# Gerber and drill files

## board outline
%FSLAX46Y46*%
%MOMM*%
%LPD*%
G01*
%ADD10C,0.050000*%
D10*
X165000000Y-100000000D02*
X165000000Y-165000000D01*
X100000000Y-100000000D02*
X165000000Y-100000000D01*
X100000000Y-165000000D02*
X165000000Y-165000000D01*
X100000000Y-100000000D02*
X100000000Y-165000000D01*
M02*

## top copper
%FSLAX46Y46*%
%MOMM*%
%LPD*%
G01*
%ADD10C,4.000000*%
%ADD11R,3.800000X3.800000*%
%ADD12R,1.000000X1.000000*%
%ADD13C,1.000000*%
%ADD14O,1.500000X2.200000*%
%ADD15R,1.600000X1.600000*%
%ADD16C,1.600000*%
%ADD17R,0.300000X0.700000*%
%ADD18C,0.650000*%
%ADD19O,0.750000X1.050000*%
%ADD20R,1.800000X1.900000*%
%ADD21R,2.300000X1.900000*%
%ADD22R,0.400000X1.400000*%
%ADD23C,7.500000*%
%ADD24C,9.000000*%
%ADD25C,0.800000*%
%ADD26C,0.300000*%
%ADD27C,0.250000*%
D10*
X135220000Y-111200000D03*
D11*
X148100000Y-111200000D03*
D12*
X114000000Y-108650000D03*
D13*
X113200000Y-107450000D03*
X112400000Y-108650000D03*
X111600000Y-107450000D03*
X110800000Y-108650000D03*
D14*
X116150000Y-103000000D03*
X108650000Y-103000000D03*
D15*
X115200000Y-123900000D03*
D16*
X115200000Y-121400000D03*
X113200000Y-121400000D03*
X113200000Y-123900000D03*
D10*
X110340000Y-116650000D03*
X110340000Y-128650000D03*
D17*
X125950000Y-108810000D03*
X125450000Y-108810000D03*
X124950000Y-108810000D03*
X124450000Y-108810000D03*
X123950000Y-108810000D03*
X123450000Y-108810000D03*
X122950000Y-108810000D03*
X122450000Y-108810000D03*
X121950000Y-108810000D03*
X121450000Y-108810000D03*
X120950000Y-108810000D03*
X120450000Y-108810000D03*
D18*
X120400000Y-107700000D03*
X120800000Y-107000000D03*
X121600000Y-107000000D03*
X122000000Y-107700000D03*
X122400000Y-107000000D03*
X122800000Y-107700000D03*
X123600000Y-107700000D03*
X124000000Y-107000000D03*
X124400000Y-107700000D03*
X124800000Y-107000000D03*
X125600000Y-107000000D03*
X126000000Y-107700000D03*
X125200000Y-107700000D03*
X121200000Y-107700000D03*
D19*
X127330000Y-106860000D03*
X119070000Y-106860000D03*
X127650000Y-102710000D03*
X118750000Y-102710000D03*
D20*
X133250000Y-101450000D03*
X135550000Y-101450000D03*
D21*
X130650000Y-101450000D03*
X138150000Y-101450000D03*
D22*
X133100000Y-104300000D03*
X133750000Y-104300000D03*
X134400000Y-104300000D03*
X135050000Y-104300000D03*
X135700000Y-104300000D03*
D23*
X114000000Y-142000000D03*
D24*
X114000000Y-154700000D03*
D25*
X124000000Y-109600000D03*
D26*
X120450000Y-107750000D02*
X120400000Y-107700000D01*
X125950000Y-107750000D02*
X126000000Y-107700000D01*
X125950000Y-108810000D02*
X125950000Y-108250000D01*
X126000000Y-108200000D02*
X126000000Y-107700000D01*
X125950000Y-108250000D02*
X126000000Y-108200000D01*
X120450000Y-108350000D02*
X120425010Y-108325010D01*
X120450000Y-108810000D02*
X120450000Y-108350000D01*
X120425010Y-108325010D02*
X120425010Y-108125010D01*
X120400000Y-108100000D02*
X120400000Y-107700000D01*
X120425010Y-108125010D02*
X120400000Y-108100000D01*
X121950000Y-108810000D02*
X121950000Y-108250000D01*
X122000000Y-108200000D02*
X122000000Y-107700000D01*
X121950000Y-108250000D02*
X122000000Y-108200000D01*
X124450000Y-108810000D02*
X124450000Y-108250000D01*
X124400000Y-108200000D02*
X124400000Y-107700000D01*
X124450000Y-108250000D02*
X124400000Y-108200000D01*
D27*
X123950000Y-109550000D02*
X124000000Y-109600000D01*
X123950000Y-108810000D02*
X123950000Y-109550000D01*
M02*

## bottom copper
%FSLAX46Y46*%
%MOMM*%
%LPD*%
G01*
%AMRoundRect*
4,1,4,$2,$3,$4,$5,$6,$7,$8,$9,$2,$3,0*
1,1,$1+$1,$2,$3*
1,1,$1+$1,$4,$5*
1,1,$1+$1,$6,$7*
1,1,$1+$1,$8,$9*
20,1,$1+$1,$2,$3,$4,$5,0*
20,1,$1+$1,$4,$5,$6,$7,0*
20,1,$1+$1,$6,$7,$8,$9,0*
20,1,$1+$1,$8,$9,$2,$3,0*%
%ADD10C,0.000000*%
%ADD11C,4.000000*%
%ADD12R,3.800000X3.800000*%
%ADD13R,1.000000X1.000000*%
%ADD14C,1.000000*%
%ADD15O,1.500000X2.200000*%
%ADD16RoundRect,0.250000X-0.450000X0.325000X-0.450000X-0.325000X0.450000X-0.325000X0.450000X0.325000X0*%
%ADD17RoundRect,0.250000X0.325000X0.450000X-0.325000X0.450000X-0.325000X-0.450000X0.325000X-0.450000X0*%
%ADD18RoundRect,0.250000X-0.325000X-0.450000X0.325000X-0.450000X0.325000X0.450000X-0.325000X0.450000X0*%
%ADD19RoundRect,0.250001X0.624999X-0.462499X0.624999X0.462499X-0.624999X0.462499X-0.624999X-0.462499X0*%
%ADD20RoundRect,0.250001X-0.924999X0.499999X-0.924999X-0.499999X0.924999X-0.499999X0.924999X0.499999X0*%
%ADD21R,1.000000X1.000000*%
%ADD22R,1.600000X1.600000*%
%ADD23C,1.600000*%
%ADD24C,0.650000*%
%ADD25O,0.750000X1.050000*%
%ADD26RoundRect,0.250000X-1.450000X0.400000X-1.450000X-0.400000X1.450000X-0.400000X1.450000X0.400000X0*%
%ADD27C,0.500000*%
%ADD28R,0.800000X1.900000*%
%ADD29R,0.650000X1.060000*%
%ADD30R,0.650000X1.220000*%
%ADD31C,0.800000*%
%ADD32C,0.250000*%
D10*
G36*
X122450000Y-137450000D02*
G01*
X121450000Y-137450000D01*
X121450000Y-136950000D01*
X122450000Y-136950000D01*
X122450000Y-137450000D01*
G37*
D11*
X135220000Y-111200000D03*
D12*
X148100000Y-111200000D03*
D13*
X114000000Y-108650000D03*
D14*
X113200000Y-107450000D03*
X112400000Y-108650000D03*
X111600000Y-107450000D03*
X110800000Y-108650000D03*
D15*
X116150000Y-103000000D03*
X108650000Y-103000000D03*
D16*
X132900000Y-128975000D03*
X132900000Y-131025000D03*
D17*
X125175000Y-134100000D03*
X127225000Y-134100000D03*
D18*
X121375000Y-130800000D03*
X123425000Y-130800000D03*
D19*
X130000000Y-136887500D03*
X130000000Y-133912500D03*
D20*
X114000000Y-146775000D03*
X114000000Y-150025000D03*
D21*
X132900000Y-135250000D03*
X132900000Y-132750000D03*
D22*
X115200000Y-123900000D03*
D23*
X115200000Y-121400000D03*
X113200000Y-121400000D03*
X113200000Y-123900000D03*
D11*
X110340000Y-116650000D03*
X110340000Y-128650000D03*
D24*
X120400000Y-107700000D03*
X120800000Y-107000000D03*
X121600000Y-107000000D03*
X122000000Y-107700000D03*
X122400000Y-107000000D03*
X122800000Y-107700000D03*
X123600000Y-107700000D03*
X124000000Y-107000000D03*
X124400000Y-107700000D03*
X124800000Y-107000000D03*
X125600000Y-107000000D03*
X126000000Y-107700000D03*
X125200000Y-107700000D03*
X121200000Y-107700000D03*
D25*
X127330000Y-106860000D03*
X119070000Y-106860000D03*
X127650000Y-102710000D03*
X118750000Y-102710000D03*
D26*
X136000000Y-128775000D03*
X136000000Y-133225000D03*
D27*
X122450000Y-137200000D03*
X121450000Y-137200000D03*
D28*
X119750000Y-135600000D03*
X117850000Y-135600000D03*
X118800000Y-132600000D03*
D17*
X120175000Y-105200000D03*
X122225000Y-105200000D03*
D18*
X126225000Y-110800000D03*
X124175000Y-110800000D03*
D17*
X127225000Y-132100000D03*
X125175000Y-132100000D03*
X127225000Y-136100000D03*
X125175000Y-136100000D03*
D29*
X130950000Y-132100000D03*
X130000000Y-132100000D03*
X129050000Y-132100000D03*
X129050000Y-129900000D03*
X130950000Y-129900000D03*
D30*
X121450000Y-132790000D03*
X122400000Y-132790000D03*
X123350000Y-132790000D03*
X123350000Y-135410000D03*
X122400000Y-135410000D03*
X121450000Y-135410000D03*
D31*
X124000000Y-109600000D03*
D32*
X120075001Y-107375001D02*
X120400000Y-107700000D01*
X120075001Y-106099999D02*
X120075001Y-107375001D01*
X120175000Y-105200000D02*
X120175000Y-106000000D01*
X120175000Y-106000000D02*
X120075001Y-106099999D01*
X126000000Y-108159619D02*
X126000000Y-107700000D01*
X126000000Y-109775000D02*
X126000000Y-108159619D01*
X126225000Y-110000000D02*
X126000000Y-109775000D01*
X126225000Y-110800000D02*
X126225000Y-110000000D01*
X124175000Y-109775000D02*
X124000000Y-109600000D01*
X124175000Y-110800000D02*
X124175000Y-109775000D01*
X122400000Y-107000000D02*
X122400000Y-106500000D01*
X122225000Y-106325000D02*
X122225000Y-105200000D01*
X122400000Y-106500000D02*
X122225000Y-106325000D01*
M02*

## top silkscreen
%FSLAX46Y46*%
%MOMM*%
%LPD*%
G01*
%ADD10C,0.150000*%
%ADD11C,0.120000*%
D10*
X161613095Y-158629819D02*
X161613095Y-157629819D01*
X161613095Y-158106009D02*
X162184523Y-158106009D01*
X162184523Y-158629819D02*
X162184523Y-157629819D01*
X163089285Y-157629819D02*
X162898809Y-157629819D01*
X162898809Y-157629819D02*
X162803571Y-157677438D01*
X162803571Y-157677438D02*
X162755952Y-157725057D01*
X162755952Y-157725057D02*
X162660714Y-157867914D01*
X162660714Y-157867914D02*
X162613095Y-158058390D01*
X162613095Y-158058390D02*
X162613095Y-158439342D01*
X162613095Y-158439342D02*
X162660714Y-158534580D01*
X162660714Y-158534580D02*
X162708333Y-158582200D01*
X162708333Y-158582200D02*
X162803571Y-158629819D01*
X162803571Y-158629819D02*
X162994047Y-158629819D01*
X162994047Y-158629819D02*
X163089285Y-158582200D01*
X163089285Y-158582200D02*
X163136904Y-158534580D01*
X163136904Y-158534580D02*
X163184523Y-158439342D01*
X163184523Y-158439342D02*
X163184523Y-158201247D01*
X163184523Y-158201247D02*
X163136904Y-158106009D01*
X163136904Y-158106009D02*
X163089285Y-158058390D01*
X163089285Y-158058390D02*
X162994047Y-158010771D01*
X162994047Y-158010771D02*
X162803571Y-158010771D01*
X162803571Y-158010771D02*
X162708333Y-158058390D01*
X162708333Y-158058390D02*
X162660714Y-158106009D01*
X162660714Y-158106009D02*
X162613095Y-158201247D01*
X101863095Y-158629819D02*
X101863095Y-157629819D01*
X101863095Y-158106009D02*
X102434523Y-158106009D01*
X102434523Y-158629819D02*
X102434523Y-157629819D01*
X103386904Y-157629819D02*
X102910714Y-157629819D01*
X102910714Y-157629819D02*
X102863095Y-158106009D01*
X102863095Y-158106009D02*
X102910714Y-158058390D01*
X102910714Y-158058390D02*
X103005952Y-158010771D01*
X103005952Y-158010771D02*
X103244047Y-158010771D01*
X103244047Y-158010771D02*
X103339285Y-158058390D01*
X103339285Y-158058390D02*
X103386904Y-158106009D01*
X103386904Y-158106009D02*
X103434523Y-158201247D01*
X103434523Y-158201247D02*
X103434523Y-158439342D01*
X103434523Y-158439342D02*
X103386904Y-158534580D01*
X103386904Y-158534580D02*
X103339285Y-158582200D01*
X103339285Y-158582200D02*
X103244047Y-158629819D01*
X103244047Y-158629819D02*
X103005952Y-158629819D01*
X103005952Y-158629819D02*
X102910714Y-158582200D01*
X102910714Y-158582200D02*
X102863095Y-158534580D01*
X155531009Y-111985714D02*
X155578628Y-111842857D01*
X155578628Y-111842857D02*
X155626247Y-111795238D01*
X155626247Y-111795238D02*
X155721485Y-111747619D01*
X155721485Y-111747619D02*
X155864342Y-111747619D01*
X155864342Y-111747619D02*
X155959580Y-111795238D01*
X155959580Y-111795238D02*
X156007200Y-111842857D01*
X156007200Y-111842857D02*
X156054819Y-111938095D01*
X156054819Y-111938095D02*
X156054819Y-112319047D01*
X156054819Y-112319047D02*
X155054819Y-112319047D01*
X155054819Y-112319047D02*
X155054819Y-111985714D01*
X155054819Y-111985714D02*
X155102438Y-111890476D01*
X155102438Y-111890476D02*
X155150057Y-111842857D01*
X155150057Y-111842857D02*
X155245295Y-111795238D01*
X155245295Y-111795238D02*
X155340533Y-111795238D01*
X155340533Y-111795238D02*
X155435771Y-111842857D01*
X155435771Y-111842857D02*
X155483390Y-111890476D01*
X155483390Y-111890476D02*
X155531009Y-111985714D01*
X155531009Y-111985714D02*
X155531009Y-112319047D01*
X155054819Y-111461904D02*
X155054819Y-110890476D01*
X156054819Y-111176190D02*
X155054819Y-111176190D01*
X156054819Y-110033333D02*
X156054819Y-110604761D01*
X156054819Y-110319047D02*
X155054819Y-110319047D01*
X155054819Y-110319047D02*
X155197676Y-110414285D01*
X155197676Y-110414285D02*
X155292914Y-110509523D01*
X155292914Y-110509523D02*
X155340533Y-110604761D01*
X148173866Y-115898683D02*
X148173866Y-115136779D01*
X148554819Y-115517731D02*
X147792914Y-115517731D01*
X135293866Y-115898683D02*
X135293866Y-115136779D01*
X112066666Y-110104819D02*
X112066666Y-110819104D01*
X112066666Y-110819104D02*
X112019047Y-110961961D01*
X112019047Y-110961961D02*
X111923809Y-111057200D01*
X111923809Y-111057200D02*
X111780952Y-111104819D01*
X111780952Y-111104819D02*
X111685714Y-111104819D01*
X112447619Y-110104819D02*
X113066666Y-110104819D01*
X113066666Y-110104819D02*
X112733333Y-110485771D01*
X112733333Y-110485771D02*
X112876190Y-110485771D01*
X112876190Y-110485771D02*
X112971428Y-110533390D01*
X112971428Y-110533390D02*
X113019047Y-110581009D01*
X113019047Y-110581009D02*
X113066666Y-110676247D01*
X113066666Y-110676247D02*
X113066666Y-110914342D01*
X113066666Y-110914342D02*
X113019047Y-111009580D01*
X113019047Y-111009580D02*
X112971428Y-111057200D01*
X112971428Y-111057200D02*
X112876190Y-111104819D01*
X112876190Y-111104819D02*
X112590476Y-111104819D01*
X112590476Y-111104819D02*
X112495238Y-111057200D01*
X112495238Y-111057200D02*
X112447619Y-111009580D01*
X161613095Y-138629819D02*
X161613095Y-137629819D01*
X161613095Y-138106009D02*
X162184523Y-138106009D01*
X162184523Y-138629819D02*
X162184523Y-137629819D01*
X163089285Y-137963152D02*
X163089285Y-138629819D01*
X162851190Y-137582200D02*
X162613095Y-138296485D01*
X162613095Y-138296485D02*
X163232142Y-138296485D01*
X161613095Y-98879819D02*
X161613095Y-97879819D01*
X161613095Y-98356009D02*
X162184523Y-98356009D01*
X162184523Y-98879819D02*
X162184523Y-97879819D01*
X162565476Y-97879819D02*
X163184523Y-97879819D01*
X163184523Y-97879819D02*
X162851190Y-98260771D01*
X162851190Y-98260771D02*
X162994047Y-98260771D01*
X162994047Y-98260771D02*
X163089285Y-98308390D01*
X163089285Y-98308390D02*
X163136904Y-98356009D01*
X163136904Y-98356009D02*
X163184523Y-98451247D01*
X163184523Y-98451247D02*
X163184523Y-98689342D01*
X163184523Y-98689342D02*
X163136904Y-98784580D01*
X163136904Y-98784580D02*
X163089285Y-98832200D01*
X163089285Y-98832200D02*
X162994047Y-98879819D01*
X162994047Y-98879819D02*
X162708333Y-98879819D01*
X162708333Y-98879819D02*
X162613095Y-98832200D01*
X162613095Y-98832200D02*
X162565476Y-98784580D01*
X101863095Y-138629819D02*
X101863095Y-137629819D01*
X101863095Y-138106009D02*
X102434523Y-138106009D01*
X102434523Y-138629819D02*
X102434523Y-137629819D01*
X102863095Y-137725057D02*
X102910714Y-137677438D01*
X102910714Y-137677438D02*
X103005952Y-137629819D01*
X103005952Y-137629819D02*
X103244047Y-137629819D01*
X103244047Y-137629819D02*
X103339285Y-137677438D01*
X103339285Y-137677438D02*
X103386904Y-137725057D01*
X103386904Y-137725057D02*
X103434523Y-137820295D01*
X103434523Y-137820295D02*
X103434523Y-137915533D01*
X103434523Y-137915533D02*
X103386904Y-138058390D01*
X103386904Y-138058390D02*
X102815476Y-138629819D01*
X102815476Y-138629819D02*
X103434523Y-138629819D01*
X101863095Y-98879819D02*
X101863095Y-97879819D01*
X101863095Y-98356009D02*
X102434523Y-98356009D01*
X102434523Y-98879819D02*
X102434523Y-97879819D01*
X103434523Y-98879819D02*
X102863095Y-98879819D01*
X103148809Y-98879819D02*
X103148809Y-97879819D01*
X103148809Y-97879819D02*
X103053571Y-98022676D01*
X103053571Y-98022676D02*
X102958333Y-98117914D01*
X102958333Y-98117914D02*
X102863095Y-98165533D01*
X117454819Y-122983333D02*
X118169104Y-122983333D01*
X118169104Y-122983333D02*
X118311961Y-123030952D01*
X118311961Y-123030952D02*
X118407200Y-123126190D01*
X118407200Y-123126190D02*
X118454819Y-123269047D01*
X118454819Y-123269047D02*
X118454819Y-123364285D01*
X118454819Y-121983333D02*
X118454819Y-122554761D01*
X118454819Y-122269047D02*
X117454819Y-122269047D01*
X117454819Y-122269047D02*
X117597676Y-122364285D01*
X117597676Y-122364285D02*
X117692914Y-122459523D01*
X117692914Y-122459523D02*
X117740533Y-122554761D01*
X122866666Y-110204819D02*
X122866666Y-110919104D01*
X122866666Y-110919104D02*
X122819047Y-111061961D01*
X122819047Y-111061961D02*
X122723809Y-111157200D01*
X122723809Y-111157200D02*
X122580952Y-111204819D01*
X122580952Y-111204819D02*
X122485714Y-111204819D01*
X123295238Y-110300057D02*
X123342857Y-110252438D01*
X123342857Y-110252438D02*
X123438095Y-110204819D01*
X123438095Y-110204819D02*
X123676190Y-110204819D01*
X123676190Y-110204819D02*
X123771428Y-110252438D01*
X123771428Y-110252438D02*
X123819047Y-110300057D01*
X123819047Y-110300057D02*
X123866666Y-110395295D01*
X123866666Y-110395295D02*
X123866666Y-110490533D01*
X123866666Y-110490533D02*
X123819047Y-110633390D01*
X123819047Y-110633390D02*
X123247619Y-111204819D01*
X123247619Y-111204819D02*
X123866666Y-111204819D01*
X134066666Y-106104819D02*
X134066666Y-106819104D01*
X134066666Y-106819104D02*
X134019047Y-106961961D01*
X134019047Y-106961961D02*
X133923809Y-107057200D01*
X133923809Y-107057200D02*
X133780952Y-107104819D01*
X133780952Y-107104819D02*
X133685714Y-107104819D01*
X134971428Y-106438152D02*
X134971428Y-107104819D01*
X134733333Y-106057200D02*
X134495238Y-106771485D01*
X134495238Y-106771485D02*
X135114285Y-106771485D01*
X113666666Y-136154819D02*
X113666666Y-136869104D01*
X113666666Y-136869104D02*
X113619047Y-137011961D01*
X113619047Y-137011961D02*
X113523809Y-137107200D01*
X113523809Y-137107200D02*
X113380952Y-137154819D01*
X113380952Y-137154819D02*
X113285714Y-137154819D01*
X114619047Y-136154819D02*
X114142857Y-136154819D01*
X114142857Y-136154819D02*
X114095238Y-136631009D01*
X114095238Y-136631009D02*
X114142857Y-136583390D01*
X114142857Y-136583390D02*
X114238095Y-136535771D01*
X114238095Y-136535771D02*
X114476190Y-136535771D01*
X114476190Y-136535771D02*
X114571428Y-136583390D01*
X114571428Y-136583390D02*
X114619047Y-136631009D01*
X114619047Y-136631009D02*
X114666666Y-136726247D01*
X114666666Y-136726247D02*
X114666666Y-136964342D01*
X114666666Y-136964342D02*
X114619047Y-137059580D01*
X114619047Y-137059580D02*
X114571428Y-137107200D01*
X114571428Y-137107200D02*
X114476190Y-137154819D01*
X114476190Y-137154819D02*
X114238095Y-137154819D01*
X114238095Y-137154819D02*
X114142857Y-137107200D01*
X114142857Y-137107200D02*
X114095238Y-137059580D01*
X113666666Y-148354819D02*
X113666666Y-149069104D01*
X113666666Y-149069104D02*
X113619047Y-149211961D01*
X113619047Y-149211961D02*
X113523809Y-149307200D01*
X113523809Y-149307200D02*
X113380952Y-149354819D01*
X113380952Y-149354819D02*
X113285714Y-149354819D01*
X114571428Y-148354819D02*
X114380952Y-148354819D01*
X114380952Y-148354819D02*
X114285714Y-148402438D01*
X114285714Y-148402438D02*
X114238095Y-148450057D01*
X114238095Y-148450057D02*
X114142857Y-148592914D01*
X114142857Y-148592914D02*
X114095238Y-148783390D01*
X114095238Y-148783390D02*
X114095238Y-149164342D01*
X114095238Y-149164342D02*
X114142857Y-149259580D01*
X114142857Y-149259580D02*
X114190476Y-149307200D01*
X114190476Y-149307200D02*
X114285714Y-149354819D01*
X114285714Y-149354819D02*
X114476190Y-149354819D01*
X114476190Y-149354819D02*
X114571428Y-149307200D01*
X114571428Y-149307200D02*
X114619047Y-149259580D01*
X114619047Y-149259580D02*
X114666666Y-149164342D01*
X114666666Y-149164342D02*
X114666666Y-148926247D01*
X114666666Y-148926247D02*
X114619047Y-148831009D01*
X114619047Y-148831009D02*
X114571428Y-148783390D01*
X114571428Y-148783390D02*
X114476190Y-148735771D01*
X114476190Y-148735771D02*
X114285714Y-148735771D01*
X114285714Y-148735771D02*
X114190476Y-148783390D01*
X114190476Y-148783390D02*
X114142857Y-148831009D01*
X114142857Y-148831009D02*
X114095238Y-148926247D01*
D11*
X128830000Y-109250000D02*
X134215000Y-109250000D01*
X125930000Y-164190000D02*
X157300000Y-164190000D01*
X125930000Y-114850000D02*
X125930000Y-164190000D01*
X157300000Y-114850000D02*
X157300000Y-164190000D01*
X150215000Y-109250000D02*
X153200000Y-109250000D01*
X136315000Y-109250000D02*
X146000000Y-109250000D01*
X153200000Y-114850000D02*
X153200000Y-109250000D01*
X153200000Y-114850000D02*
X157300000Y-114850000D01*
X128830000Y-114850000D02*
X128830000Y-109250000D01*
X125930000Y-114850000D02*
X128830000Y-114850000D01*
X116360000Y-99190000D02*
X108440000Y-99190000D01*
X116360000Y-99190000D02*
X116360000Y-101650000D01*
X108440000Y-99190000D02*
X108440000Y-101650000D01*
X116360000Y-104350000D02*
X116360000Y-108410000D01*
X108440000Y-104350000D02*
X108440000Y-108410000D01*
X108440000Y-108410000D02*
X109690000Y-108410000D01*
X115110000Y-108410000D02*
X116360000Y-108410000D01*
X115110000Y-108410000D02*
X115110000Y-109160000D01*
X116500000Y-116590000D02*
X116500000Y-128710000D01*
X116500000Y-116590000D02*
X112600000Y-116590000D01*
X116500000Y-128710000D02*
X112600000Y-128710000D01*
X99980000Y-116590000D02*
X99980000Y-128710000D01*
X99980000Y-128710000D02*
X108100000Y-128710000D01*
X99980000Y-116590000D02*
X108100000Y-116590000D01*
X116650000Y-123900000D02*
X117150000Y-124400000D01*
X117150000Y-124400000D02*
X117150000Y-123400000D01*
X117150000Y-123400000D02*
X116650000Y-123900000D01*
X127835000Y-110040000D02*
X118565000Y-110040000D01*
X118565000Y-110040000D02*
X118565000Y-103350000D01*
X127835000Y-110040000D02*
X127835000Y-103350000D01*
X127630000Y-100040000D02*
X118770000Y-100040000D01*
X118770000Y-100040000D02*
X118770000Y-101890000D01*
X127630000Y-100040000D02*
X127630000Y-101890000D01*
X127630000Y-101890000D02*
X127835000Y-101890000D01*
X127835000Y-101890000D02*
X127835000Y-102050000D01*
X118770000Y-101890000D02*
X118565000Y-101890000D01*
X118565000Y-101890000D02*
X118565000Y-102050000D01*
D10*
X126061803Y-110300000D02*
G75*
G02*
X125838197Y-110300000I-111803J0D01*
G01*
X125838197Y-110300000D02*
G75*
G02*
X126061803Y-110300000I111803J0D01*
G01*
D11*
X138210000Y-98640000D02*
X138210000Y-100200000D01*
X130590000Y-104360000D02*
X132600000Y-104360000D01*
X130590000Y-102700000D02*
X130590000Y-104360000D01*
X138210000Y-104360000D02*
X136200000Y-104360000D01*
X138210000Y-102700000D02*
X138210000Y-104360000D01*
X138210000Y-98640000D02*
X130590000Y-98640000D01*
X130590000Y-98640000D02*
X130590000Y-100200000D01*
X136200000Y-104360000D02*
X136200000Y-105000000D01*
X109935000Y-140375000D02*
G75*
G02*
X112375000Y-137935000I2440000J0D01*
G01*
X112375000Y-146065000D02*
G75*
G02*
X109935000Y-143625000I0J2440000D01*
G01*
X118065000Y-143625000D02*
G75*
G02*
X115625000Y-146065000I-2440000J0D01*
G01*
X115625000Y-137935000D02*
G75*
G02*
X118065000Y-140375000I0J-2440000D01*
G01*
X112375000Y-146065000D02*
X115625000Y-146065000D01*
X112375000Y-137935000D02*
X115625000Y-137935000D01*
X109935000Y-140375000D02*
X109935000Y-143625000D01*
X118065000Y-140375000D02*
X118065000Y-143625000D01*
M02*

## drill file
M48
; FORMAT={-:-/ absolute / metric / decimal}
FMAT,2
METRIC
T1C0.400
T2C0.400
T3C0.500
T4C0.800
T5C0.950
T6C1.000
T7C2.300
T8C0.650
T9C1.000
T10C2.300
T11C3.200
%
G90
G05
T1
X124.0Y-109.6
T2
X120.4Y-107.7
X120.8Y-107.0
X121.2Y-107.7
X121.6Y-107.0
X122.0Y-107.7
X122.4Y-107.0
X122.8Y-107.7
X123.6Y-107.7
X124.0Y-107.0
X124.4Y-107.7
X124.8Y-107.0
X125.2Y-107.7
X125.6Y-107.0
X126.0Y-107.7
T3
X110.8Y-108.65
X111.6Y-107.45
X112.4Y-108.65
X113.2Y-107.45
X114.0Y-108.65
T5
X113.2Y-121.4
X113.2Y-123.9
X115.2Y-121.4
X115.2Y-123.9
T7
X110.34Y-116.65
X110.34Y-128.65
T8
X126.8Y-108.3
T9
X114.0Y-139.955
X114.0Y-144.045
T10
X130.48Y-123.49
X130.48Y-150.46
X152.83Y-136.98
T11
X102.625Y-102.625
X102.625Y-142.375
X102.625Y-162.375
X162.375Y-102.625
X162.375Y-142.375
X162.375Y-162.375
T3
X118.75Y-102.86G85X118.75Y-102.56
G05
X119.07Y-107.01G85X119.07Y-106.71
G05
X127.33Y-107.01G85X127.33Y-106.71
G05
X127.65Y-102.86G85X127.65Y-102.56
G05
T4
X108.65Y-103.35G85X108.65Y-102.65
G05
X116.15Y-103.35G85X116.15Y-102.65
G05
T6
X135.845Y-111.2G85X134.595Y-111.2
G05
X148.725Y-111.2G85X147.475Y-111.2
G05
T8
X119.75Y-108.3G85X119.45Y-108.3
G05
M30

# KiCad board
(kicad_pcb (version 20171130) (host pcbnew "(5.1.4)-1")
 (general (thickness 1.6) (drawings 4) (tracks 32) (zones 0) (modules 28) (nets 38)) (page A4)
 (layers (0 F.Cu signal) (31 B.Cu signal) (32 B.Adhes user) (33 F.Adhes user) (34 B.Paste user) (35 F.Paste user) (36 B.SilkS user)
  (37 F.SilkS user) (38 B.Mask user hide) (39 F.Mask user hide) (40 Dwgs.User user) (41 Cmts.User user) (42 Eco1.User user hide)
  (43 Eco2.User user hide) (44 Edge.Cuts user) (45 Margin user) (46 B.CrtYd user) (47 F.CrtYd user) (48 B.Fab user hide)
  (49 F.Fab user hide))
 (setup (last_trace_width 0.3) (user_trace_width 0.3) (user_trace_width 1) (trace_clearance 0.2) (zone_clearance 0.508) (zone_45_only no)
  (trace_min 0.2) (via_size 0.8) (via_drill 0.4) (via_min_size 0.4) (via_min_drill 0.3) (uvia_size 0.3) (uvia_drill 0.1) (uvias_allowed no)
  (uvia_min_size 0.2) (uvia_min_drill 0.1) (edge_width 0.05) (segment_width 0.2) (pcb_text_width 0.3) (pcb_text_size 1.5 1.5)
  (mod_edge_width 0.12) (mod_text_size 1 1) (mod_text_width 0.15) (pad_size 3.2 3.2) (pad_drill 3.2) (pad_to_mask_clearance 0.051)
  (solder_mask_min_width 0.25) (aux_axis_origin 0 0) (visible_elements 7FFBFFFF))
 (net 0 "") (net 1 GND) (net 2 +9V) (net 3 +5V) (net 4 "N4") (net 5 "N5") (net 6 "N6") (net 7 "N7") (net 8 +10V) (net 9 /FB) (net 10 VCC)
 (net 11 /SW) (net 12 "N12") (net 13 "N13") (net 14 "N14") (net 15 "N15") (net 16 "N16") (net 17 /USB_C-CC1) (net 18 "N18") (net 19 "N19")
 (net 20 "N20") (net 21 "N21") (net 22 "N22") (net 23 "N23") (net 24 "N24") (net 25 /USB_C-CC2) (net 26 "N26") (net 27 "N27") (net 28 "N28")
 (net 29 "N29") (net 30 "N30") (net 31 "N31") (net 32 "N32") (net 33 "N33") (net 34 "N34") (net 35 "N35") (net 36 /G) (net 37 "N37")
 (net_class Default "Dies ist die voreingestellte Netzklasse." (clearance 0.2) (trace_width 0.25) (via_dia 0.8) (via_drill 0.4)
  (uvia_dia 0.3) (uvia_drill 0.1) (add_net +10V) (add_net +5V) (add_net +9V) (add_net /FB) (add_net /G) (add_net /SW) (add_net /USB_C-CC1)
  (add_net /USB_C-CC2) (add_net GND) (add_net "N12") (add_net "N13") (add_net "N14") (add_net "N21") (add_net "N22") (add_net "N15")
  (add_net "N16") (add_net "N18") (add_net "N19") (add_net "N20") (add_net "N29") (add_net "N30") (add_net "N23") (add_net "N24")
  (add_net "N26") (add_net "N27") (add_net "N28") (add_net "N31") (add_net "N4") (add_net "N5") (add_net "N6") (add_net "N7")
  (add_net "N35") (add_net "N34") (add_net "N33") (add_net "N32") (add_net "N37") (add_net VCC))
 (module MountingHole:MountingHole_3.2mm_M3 (layer F.Cu) (at 162.375 162.375)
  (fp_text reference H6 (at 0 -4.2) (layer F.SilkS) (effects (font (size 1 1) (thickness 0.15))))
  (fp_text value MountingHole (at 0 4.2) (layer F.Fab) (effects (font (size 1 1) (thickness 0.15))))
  (pad 1 np_thru_hole circle (at 0 0) (size 3.2 3.2) (drill 3.2) (layers *.Cu *.Mask)))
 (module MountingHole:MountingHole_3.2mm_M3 (layer F.Cu) (at 102.625 162.375)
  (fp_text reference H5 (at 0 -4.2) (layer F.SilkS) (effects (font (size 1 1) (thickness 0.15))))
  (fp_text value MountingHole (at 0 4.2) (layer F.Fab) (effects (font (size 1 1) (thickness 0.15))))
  (pad 1 np_thru_hole circle (at 0 0) (size 3.2 3.2) (drill 3.2) (layers *.Cu *.Mask)))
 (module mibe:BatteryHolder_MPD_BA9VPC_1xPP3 (layer F.Cu) (at 148.1 111.2 270)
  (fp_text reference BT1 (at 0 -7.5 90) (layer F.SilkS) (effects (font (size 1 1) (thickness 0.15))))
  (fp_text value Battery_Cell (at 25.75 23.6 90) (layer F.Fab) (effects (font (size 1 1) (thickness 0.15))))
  (fp_line (start -1.95 19.27) (end -1.95 13.885) (layer F.SilkS) (width 0.12))
  (fp_line (start 52.99 22.17) (end 52.99 -9.2) (layer F.SilkS) (width 0.12))
  (fp_line (start 3.65 22.17) (end 52.99 22.17) (layer F.SilkS) (width 0.12))
  (fp_line (start 3.65 -9.2) (end 52.99 -9.2) (layer F.SilkS) (width 0.12))
  (fp_line (start -1.95 -2.115) (end -1.95 -5.1) (layer F.SilkS) (width 0.12))
  (fp_line (start -1.95 11.785) (end -1.95 2.1) (layer F.SilkS) (width 0.12))
  (fp_line (start 3.65 -5.1) (end -1.95 -5.1) (layer F.SilkS) (width 0.12))
  (fp_line (start 3.65 -5.1) (end 3.65 -9.2) (layer F.SilkS) (width 0.12))
  (fp_line (start 3.65 19.27) (end -1.95 19.27) (layer F.SilkS) (width 0.12))
  (fp_line (start 3.65 22.17) (end 3.65 19.27) (layer F.SilkS) (width 0.12))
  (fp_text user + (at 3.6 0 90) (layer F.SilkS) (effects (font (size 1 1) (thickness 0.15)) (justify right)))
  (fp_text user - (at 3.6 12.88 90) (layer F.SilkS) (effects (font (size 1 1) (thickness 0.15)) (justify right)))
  (pad "" np_thru_hole circle (at 39.26 17.62 270) (size 2.3 2.3) (drill 2.3) (layers *.Cu *.Mask))
  (pad "" np_thru_hole circle (at 12.29 17.62 270) (size 2.3 2.3) (drill 2.3) (layers *.Cu *.Mask))
  (pad "" np_thru_hole circle (at 25.78 -4.73 270) (size 2.3 2.3) (drill 2.3) (layers *.Cu *.Mask))
  (pad 2 thru_hole circle (at 0 12.88 270) (size 4 4) (drill oval 1 2.25) (layers *.Cu *.Mask) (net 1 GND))
  (pad 1 thru_hole rect (at 0 0 270) (size 3.8 3.8) (drill oval 1 2.25) (layers *.Cu *.Mask) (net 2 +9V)))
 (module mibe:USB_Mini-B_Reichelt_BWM (layer F.Cu) (at 114 108.65 180)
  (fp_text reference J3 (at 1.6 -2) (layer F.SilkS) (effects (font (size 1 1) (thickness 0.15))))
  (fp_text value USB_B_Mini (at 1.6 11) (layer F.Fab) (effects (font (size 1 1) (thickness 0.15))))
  (fp_line (start -2.36 9.46) (end 5.56 9.46) (layer F.SilkS) (width 0.12))
  (fp_line (start -2.36 9.46) (end -2.36 7) (layer F.SilkS) (width 0.12))
  (fp_line (start 5.56 9.46) (end 5.56 7) (layer F.SilkS) (width 0.12))
  (fp_line (start -2.36 4.3) (end -2.36 0.24) (layer F.SilkS) (width 0.12))
  (fp_line (start 5.56 4.3) (end 5.56 0.24) (layer F.SilkS) (width 0.12))
  (fp_line (start 5.56 0.24) (end 4.31 0.24) (layer F.SilkS) (width 0.12))
  (fp_line (start -1.11 0.24) (end -2.36 0.24) (layer F.SilkS) (width 0.12))
  (fp_line (start -1.11 0.24) (end -1.11 -0.51) (layer F.SilkS) (width 0.12))
  (pad 1 thru_hole rect (at 0 0 180) (size 1 1) (drill 0.5) (layers *.Cu *.Mask) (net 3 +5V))
  (pad 2 thru_hole circle (at 0.8 1.2 180) (size 1 1) (drill 0.5) (layers *.Cu *.Mask) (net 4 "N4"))
  (pad 3 thru_hole circle (at 1.6 0 180) (size 1 1) (drill 0.5) (layers *.Cu *.Mask) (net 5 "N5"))
  (pad 4 thru_hole circle (at 2.4 1.2 180) (size 1 1) (drill 0.5) (layers *.Cu *.Mask) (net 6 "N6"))
  (pad 5 thru_hole circle (at 3.2 0 180) (size 1 1) (drill 0.5) (layers *.Cu *.Mask) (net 1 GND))
  (pad 6 thru_hole oval (at -2.15 5.65 180) (size 1.5 2.2) (drill oval 0.8 1.5) (layers *.Cu *.Mask) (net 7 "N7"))
  (pad 6 thru_hole oval (at 5.35 5.65 180) (size 1.5 2.2) (drill oval 0.8 1.5) (layers *.Cu *.Mask) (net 7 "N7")))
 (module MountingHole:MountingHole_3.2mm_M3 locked (layer F.Cu) (at 162.375 142.375)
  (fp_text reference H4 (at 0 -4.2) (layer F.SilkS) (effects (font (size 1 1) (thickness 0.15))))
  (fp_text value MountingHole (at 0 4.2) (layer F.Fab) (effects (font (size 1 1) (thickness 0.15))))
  (pad 1 np_thru_hole circle (at 0 0) (size 3.2 3.2) (drill 3.2) (layers *.Cu *.Mask)))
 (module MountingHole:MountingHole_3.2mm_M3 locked (layer F.Cu) (at 162.375 102.625)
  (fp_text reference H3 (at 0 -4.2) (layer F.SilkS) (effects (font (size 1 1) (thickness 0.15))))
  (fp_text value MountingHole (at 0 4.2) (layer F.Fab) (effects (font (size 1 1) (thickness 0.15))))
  (pad 1 np_thru_hole circle (at 0 0) (size 3.2 3.2) (drill 3.2) (layers *.Cu *.Mask)))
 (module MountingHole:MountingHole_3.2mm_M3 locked (layer F.Cu) (at 102.625 142.375)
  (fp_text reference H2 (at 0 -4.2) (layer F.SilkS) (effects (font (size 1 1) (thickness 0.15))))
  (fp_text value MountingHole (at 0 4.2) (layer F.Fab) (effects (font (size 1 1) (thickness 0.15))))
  (pad 1 np_thru_hole circle (at 0 0) (size 3.2 3.2) (drill 3.2) (layers *.Cu *.Mask)))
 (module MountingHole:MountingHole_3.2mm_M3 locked (layer F.Cu) (at 102.625 102.625)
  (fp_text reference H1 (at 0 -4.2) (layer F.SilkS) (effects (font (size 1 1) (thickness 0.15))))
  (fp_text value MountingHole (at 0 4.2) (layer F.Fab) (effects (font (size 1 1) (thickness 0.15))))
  (pad 1 np_thru_hole circle (at 0 0) (size 3.2 3.2) (drill 3.2) (layers *.Cu *.Mask)))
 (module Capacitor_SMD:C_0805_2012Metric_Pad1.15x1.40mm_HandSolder (layer B.Cu) (at 132.9 130 270)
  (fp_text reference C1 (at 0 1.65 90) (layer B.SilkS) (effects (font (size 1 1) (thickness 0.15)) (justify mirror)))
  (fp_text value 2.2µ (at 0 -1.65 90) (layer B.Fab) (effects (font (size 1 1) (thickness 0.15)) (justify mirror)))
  (pad 1 smd roundrect (at -1.025 0 270) (size 1.15 1.4) (layers B.Cu B.Paste B.Mask) (roundrect_rratio 0.217391) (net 3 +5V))
  (pad 2 smd roundrect (at 1.025 0 270) (size 1.15 1.4) (layers B.Cu B.Paste B.Mask) (roundrect_rratio 0.217391) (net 1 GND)))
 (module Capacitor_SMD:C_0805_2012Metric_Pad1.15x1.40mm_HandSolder (layer B.Cu) (at 126.2 134.1 180)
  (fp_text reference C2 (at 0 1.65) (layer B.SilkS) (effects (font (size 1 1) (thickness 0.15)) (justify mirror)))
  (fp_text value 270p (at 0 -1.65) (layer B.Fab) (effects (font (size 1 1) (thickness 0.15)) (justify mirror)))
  (pad 2 smd roundrect (at 1.025 0 180) (size 1.15 1.4) (layers B.Cu B.Paste B.Mask) (roundrect_rratio 0.217391) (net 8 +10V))
  (pad 1 smd roundrect (at -1.025 0 180) (size 1.15 1.4) (layers B.Cu B.Paste B.Mask) (roundrect_rratio 0.217391) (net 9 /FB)))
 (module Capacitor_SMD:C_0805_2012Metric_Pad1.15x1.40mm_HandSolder (layer B.Cu) (at 122.4 130.8)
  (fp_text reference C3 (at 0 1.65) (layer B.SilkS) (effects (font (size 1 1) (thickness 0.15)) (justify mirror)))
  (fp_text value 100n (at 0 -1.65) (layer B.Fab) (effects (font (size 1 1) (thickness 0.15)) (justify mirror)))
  (pad 1 smd roundrect (at -1.025 0) (size 1.15 1.4) (layers B.Cu B.Paste B.Mask) (roundrect_rratio 0.217391) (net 2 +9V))
  (pad 2 smd roundrect (at 1.025 0) (size 1.15 1.4) (layers B.Cu B.Paste B.Mask) (roundrect_rratio 0.217391) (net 1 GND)))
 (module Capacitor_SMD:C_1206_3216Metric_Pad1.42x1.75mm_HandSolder (layer B.Cu) (at 130 135.4 90)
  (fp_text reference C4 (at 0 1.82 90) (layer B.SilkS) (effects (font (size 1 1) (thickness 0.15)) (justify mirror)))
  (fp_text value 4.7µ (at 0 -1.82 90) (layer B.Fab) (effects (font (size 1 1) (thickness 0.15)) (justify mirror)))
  (pad 1 smd roundrect (at -1.4875 0 90) (size 1.425 1.75) (layers B.Cu B.Paste B.Mask) (roundrect_rratio 0.175439) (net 8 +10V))
  (pad 2 smd roundrect (at 1.4875 0 90) (size 1.425 1.75) (layers B.Cu B.Paste B.Mask) (roundrect_rratio 0.175439) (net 1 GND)))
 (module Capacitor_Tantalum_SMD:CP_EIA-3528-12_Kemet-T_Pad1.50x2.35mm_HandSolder (layer B.Cu) (at 114 148.4 270)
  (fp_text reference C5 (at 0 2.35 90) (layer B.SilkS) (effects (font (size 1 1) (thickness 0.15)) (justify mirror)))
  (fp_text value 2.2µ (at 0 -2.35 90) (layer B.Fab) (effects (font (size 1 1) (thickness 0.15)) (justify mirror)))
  (pad 1 smd roundrect (at -1.625 0 270) (size 1.5 2.35) (layers B.Cu B.Paste B.Mask) (roundrect_rratio 0.166667) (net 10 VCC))
  (pad 2 smd roundrect (at 1.625 0 270) (size 1.5 2.35) (layers B.Cu B.Paste B.Mask) (roundrect_rratio 0.166667) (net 1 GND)))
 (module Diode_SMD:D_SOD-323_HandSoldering (layer B.Cu) (at 132.9 134 90)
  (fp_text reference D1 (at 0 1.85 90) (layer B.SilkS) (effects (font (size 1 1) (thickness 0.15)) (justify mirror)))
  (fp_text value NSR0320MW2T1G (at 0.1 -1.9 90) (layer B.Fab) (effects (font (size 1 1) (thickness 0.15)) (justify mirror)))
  (pad 1 smd rect (at -1.25 0 90) (size 1 1) (layers B.Cu B.Paste B.Mask) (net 8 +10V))
  (pad 2 smd rect (at 1.25 0 90) (size 1 1) (layers B.Cu B.Paste B.Mask) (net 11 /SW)))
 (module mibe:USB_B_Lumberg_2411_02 (layer F.Cu) (at 115.2 123.9 270)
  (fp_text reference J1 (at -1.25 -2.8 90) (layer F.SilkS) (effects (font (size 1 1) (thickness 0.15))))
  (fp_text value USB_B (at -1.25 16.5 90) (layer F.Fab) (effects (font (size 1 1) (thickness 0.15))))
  (fp_line (start -7.31 -1.3) (end 4.81 -1.3) (layer F.SilkS) (width 0.12))
  (fp_line (start -7.31 -1.3) (end -7.31 2.6) (layer F.SilkS) (width 0.12))
  (fp_line (start 4.81 -1.3) (end 4.81 2.6) (layer F.SilkS) (width 0.12))
  (fp_line (start -7.31 15.22) (end 4.81 15.22) (layer F.SilkS) (width 0.12))
  (fp_line (start 4.81 15.22) (end 4.81 7.1) (layer F.SilkS) (width 0.12))
  (fp_line (start -7.31 15.22) (end -7.31 7.1) (layer F.SilkS) (width 0.12))
  (fp_line (start 0 -1.45) (end 0.5 -1.95) (layer F.SilkS) (width 0.12))
  (fp_line (start 0.5 -1.95) (end -0.5 -1.95) (layer F.SilkS) (width 0.12))
  (fp_line (start -0.5 -1.95) (end 0 -1.45) (layer F.SilkS) (width 0.12))
  (pad 1 thru_hole rect (at 0 0 270) (size 1.6 1.6) (drill 0.95) (layers *.Cu *.Mask) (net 3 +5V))
  (pad 2 thru_hole circle (at -2.5 0 270) (size 1.6 1.6) (drill 0.95) (layers *.Cu *.Mask) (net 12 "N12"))
  (pad 3 thru_hole circle (at -2.5 2 270) (size 1.6 1.6) (drill 0.95) (layers *.Cu *.Mask) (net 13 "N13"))
  (pad 4 thru_hole circle (at 0 2 270) (size 1.6 1.6) (drill 0.95) (layers *.Cu *.Mask) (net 1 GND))
  (pad 5 thru_hole circle (at -7.25 4.86 270) (size 4 4) (drill 2.3) (layers *.Cu *.Mask) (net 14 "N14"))
  (pad 5 thru_hole circle (at 4.75 4.86 270) (size 4 4) (drill 2.3) (layers *.Cu *.Mask) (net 14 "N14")))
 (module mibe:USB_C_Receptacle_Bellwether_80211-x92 (layer F.Cu) (at 123.2 108.3 180)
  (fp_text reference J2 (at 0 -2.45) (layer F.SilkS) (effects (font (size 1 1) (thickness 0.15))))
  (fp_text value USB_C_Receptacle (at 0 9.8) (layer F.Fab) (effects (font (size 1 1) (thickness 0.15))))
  (fp_line (start -4.635 -1.74) (end 4.635 -1.74) (layer F.SilkS) (width 0.12))
  (fp_line (start 4.635 -1.74) (end 4.635 4.95) (layer F.SilkS) (width 0.12))
  (fp_line (start -4.635 -1.74) (end -4.635 4.95) (layer F.SilkS) (width 0.12))
  (fp_line (start -4.43 8.26) (end 4.43 8.26) (layer F.SilkS) (width 0.12))
  (fp_line (start 4.43 8.26) (end 4.43 6.41) (layer F.SilkS) (width 0.12))
  (fp_line (start -4.43 8.26) (end -4.43 6.41) (layer F.SilkS) (width 0.12))
  (fp_line (start -4.43 6.41) (end -4.635 6.41) (layer F.SilkS) (width 0.12))
  (fp_line (start -4.635 6.41) (end -4.635 6.25) (layer F.SilkS) (width 0.12))
  (fp_line (start 4.43 6.41) (end 4.635 6.41) (layer F.SilkS) (width 0.12))
  (fp_line (start 4.635 6.41) (end 4.635 6.25) (layer F.SilkS) (width 0.12))
  (fp_circle (center -2.75 -2) (end -2.638197 -2) (layer F.SilkS) (width 0.15))
  (pad A1 smd rect (at -2.75 -0.51 180) (size 0.3 0.7) (layers F.Cu F.Paste F.Mask) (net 1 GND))
  (pad A2 smd rect (at -2.25 -0.51 180) (size 0.3 0.7) (layers F.Cu F.Paste F.Mask) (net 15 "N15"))
  (pad A3 smd rect (at -1.75 -0.51 180) (size 0.3 0.7) (layers F.Cu F.Paste F.Mask) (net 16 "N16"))
  (pad A4 smd rect (at -1.25 -0.51 180) (size 0.3 0.7) (layers F.Cu F.Paste F.Mask) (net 3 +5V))
  (pad A5 smd rect (at -0.75 -0.51 180) (size 0.3 0.7) (layers F.Cu F.Paste F.Mask) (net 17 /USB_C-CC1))
  (pad A6 smd rect (at -0.25 -0.51 180) (size 0.3 0.7) (layers F.Cu F.Paste F.Mask) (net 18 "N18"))
  (pad A7 smd rect (at 0.25 -0.51 180) (size 0.3 0.7) (layers F.Cu F.Paste F.Mask) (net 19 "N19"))
  (pad A8 smd rect (at 0.75 -0.51 180) (size 0.3 0.7) (layers F.Cu F.Paste F.Mask) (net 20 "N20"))
  (pad A9 smd rect (at 1.25 -0.51 180) (size 0.3 0.7) (layers F.Cu F.Paste F.Mask) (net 3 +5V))
  (pad A10 smd rect (at 1.75 -0.51 180) (size 0.3 0.7) (layers F.Cu F.Paste F.Mask) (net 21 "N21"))
  (pad A11 smd rect (at 2.25 -0.51 180) (size 0.3 0.7) (layers F.Cu F.Paste F.Mask) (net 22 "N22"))
  (pad A12 smd rect (at 2.75 -0.51 180) (size 0.3 0.7) (layers F.Cu F.Paste F.Mask) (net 1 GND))
  (pad B1 thru_hole circle (at 2.8 0.6 180) (size 0.65 0.65) (drill 0.4) (layers *.Cu *.Mask) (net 1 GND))
  (pad B2 thru_hole circle (at 2.4 1.3 180) (size 0.65 0.65) (drill 0.4) (layers *.Cu *.Mask) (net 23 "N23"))
  (pad B3 thru_hole circle (at 1.6 1.3 180) (size 0.65 0.65) (drill 0.4) (layers *.Cu *.Mask) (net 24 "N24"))
  (pad B4 thru_hole circle (at 1.2 0.6 180) (size 0.65 0.65) (drill 0.4) (layers *.Cu *.Mask) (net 3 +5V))
  (pad B5 thru_hole circle (at 0.8 1.3 180) (size 0.65 0.65) (drill 0.4) (layers *.Cu *.Mask) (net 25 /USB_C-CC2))
  (pad B6 thru_hole circle (at 0.4 0.6 180) (size 0.65 0.65) (drill 0.4) (layers *.Cu *.Mask) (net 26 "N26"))
  (pad B7 thru_hole circle (at -0.4 0.6 180) (size 0.65 0.65) (drill 0.4) (layers *.Cu *.Mask) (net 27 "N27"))
  (pad B8 thru_hole circle (at -0.8 1.3 180) (size 0.65 0.65) (drill 0.4) (layers *.Cu *.Mask) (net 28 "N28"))
  (pad B9 thru_hole circle (at -1.2 0.6 180) (size 0.65 0.65) (drill 0.4) (layers *.Cu *.Mask) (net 3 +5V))
  (pad B10 thru_hole circle (at -1.6 1.3 180) (size 0.65 0.65) (drill 0.4) (layers *.Cu *.Mask) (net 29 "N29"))
  (pad B11 thru_hole circle (at -2.4 1.3 180) (size 0.65 0.65) (drill 0.4) (layers *.Cu *.Mask) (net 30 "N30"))
  (pad B12 thru_hole circle (at -2.8 0.6 180) (size 0.65 0.65) (drill 0.4) (layers *.Cu *.Mask) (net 1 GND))
  (pad "" thru_hole circle (at -2 0.6 180) (size 0.65 0.65) (drill 0.4) (layers *.Cu *.Mask))
  (pad "" thru_hole circle (at 2 0.6 180) (size 0.65 0.65) (drill 0.4) (layers *.Cu *.Mask))
  (pad "" np_thru_hole circle (at -3.6 0 180) (size 0.65 0.65) (drill 0.65) (layers *.Cu *.Mask))
  (pad "" np_thru_hole oval (at 3.6 0 180) (size 0.95 0.65) (drill oval 0.95 0.65) (layers *.Cu *.Mask))
  (pad S1 thru_hole oval (at -4.13 1.44 180) (size 0.75 1.05) (drill oval 0.5 0.8) (layers *.Cu *.Mask) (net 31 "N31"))
  (pad S1 thru_hole oval (at 4.13 1.44 180) (size 0.75 1.05) (drill oval 0.5 0.8) (layers *.Cu *.Mask) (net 31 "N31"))
  (pad S1 thru_hole oval (at -4.45 5.59 180) (size 0.75 1.05) (drill oval 0.5 0.8) (layers *.Cu *.Mask) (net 31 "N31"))
  (pad S1 thru_hole oval (at 4.45 5.59 180) (size 0.75 1.05) (drill oval 0.5 0.8) (layers *.Cu *.Mask) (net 31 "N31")))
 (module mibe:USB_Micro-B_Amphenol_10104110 (layer F.Cu) (at 134.4 104.3 180)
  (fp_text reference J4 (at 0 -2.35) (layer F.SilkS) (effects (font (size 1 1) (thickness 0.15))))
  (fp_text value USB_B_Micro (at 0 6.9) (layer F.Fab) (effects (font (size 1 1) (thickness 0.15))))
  (fp_line (start -3.81 5.66) (end -3.81 4.1) (layer F.SilkS) (width 0.12))
  (fp_line (start 3.81 -0.06) (end 1.8 -0.06) (layer F.SilkS) (width 0.12))
  (fp_line (start 3.81 1.6) (end 3.81 -0.06) (layer F.SilkS) (width 0.12))
  (fp_line (start -3.81 -0.06) (end -1.8 -0.06) (layer F.SilkS) (width 0.12))
  (fp_line (start -3.81 1.6) (end -3.81 -0.06) (layer F.SilkS) (width 0.12))
  (fp_line (start -3.81 5.66) (end 3.81 5.66) (layer F.SilkS) (width 0.12))
  (fp_line (start 3.81 5.66) (end 3.81 4.1) (layer F.SilkS) (width 0.12))
  (fp_line (start -1.8 -0.06) (end -1.8 -0.7) (layer F.SilkS) (width 0.12))
  (pad 6 smd rect (at 1.15 2.85 180) (size 1.8 1.9) (layers F.Cu F.Paste F.Mask) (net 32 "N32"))
  (pad 6 smd rect (at -1.15 2.85 180) (size 1.8 1.9) (layers F.Cu F.Paste F.Mask) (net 32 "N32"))
  (pad 6 smd rect (at 3.75 2.85 180) (size 2.3 1.9) (layers F.Cu F.Paste F.Mask) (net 32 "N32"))
  (pad 6 smd rect (at -3.75 2.85 180) (size 2.3 1.9) (layers F.Cu F.Paste F.Mask) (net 32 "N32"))
  (pad 5 smd rect (at 1.3 0 180) (size 0.4 1.4) (layers F.Cu F.Paste F.Mask) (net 1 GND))
  (pad 4 smd rect (at 0.65 0 180) (size 0.4 1.4) (layers F.Cu F.Paste F.Mask) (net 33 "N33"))
  (pad 3 smd rect (at 0 0 180) (size 0.4 1.4) (layers F.Cu F.Paste F.Mask) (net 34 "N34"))
  (pad 2 smd rect (at -0.65 0 180) (size 0.4 1.4) (layers F.Cu F.Paste F.Mask) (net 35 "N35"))
  (pad 1 smd rect (at -1.3 0 180) (size 0.4 1.4) (layers F.Cu F.Paste F.Mask) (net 3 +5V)))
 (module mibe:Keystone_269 (layer F.Cu) (at 114 142)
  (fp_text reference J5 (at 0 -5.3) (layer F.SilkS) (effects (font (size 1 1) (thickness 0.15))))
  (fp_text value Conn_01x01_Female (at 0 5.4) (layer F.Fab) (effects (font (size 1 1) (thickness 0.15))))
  (fp_arc (start -1.625 -1.625) (end -4.065 -1.625) (angle 90) (layer F.SilkS) (width 0.12))
  (fp_arc (start -1.625 1.625) (end -1.625 4.065) (angle 90) (layer F.SilkS) (width 0.12))
  (fp_arc (start 1.625 1.625) (end 4.065 1.625) (angle 90) (layer F.SilkS) (width 0.12))
  (fp_arc (start 1.625 -1.625) (end 1.625 -4.065) (angle 90) (layer F.SilkS) (width 0.12))
  (fp_line (start -1.625 4.065) (end 1.625 4.065) (layer F.SilkS) (width 0.12))
  (fp_line (start -1.625 -4.065) (end 1.625 -4.065) (layer F.SilkS) (width 0.12))
  (fp_line (start -4.065 -1.625) (end -4.065 1.625) (layer F.SilkS) (width 0.12))
  (fp_line (start 4.065 -1.625) (end 4.065 1.625) (layer F.SilkS) (width 0.12))
  (pad "" np_thru_hole circle (at 0 2.045) (size 1 1) (drill 1) (layers *.Cu *.Mask))
  (pad "" np_thru_hole circle (at 0 -2.045) (size 1 1) (drill 1) (layers *.Cu *.Mask))
  (pad 1 smd circle (at 0 0) (size 7.5 7.5) (layers F.Cu F.Paste F.Mask) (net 10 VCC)))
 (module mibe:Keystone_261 (layer F.Cu) (at 114 154.7)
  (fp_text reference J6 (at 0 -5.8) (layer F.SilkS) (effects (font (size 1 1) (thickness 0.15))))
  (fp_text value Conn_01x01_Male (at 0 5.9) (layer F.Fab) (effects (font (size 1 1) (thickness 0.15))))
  (pad 1 smd circle (at 0 0) (size 9 9) (layers F.Cu F.Paste F.Mask) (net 1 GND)))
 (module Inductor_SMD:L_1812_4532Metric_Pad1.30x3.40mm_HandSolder (layer B.Cu) (at 136 131 270)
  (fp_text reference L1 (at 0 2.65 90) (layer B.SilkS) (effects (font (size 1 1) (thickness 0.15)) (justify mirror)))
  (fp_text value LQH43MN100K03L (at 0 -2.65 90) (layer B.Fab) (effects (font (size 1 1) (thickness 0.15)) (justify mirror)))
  (pad 1 smd roundrect (at -2.225 0 270) (size 1.3 3.4) (layers B.Cu B.Paste B.Mask) (roundrect_rratio 0.192308) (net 3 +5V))
  (pad 2 smd roundrect (at 2.225 0 270) (size 1.3 3.4) (layers B.Cu B.Paste B.Mask) (roundrect_rratio 0.192308) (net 11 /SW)))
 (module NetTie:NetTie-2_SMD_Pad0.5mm (layer B.Cu) (at 121.95 137.2 180)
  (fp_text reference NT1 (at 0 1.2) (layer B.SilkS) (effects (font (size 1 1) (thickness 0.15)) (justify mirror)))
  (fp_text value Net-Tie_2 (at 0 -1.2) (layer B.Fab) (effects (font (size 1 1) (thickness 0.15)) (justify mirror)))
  (fp_poly (pts (xy -0.5 0.25) (xy 0.5 0.25) (xy 0.5 -0.25) (xy -0.5 -0.25)) (layer B.Cu) (width 0))
  (pad 1 smd circle (at -0.5 0 180) (size 0.5 0.5) (layers B.Cu) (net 8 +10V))
  (pad 2 smd circle (at 0.5 0 180) (size 0.5 0.5) (layers B.Cu) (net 10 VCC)))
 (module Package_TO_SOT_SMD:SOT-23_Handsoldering (layer B.Cu) (at 118.8 134.1 90)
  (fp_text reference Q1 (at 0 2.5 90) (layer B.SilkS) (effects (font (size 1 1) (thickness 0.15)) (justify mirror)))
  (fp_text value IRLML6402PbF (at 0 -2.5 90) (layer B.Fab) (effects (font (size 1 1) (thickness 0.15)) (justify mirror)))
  (pad 1 smd rect (at -1.5 0.95 90) (size 1.9 0.8) (layers B.Cu B.Paste B.Mask) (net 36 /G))
  (pad 2 smd rect (at -1.5 -0.95 90) (size 1.9 0.8) (layers B.Cu B.Paste B.Mask) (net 10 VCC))
  (pad 3 smd rect (at 1.5 0 90) (size 1.9 0.8) (layers B.Cu B.Paste B.Mask) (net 2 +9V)))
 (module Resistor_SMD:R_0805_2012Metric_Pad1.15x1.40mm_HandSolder (layer B.Cu) (at 121.2 105.2 180)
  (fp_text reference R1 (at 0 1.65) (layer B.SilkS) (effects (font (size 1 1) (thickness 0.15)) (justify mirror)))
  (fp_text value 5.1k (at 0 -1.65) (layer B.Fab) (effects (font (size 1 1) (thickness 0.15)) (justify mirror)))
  (pad 2 smd roundrect (at 1.025 0 180) (size 1.15 1.4) (layers B.Cu B.Paste B.Mask) (roundrect_rratio 0.217391) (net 1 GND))
  (pad 1 smd roundrect (at -1.025 0 180) (size 1.15 1.4) (layers B.Cu B.Paste B.Mask) (roundrect_rratio 0.217391) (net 25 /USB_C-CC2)))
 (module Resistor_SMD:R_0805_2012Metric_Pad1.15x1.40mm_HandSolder (layer B.Cu) (at 125.2 110.8)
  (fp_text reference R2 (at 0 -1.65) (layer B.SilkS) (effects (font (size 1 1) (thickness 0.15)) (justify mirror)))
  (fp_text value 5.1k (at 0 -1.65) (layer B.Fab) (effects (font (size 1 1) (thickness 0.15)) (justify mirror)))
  (pad 2 smd roundrect (at 1.025 0) (size 1.15 1.4) (layers B.Cu B.Paste B.Mask) (roundrect_rratio 0.217391) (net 1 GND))
  (pad 1 smd roundrect (at -1.025 0) (size 1.15 1.4) (layers B.Cu B.Paste B.Mask) (roundrect_rratio 0.217391) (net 17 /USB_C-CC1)))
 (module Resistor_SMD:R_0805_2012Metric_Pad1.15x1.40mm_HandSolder (layer B.Cu) (at 126.2 132.1 180)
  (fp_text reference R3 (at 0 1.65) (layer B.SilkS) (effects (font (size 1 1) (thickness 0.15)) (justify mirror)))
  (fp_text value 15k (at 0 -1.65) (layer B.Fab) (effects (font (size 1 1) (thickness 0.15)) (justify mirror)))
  (pad 1 smd roundrect (at -1.025 0 180) (size 1.15 1.4) (layers B.Cu B.Paste B.Mask) (roundrect_rratio 0.217391) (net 9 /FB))
  (pad 2 smd roundrect (at 1.025 0 180) (size 1.15 1.4) (layers B.Cu B.Paste B.Mask) (roundrect_rratio 0.217391) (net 1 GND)))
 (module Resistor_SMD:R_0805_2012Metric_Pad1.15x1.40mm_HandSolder (layer B.Cu) (at 126.2 136.1 180)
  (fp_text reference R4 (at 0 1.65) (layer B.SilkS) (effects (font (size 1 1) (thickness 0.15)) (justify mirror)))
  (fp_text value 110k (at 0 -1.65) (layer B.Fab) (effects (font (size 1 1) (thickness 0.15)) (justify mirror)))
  (pad 1 smd roundrect (at -1.025 0 180) (size 1.15 1.4) (layers B.Cu B.Paste B.Mask) (roundrect_rratio 0.217391) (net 9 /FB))
  (pad 2 smd roundrect (at 1.025 0 180) (size 1.15 1.4) (layers B.Cu B.Paste B.Mask) (roundrect_rratio 0.217391) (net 8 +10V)))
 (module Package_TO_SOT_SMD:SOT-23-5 (layer B.Cu) (at 130 131 90)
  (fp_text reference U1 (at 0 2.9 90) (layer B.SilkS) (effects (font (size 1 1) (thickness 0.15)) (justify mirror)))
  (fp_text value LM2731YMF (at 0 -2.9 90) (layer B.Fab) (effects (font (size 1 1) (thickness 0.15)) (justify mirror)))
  (pad 1 smd rect (at -1.1 0.95 90) (size 1.06 0.65) (layers B.Cu B.Paste B.Mask) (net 11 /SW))
  (pad 2 smd rect (at -1.1 0 90) (size 1.06 0.65) (layers B.Cu B.Paste B.Mask) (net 1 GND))
  (pad 3 smd rect (at -1.1 -0.95 90) (size 1.06 0.65) (layers B.Cu B.Paste B.Mask) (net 9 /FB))
  (pad 4 smd rect (at 1.1 -0.95 90) (size 1.06 0.65) (layers B.Cu B.Paste B.Mask) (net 3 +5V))
  (pad 5 smd rect (at 1.1 0.95 90) (size 1.06 0.65) (layers B.Cu B.Paste B.Mask) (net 3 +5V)))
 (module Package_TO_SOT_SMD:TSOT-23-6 (layer B.Cu) (at 122.4 134.1 270)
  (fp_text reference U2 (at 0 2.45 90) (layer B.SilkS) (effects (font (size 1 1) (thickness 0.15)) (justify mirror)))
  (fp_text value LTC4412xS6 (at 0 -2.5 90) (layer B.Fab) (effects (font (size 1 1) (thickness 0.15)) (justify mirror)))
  (pad 1 smd rect (at -1.31 0.95 270) (size 1.22 0.65) (layers B.Cu B.Paste B.Mask) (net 2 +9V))
  (pad 2 smd rect (at -1.31 0 270) (size 1.22 0.65) (layers B.Cu B.Paste B.Mask) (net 1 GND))
  (pad 3 smd rect (at -1.31 -0.95 270) (size 1.22 0.65) (layers B.Cu B.Paste B.Mask) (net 1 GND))
  (pad 4 smd rect (at 1.31 -0.95 270) (size 1.22 0.65) (layers B.Cu B.Paste B.Mask) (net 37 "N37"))
  (pad 5 smd rect (at 1.31 0 270) (size 1.22 0.65) (layers B.Cu B.Paste B.Mask) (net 36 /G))
  (pad 6 smd rect (at 1.31 0.95 270) (size 1.22 0.65) (layers B.Cu B.Paste B.Mask) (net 10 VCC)))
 (gr_line (start 165 100) (end 165 165) (layer Edge.Cuts) (width 0.05))
 (gr_line (start 100 100) (end 165 100) (layer Edge.Cuts) (width 0.05))
 (gr_line (start 100 165) (end 165 165) (layer Edge.Cuts) (width 0.05))
 (gr_line (start 100 100) (end 100 165) (layer Edge.Cuts) (width 0.05))
 (segment (start 120.45 107.75) (end 120.4 107.7) (width 0.3) (layer F.Cu) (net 1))
 (segment (start 125.95 107.75) (end 126 107.7) (width 0.3) (layer F.Cu) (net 1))
 (segment (start 120.075001 107.375001) (end 120.4 107.7) (width 0.25) (layer B.Cu) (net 1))
 (segment (start 120.075001 106.099999) (end 120.075001 107.375001) (width 0.25) (layer B.Cu) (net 1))
 (segment (start 120.175 105.2) (end 120.175 106) (width 0.25) (layer B.Cu) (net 1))
 (segment (start 120.175 106) (end 120.075001 106.099999) (width 0.25) (layer B.Cu) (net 1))
 (segment (start 126 108.159619) (end 126 107.7) (width 0.25) (layer B.Cu) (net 1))
 (segment (start 126 109.775) (end 126 108.159619) (width 0.25) (layer B.Cu) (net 1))
 (segment (start 126.225 110) (end 126 109.775) (width 0.25) (layer B.Cu) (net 1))
 (segment (start 126.225 110.8) (end 126.225 110) (width 0.25) (layer B.Cu) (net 1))
 (segment (start 125.95 108.81) (end 125.95 108.25) (width 0.3) (layer F.Cu) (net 1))
 (segment (start 126 108.2) (end 126 107.7) (width 0.3) (layer F.Cu) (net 1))
 (segment (start 125.95 108.25) (end 126 108.2) (width 0.3) (layer F.Cu) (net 1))
 (segment (start 120.45 108.35) (end 120.42501 108.32501) (width 0.3) (layer F.Cu) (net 1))
 (segment (start 120.45 108.81) (end 120.45 108.35) (width 0.3) (layer F.Cu) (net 1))
 (segment (start 120.42501 108.32501) (end 120.42501 108.12501) (width 0.3) (layer F.Cu) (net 1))
 (segment (start 120.4 108.1) (end 120.4 107.7) (width 0.3) (layer F.Cu) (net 1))
 (segment (start 120.42501 108.12501) (end 120.4 108.1) (width 0.3) (layer F.Cu) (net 1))
 (segment (start 121.95 108.81) (end 121.95 108.25) (width 0.3) (layer F.Cu) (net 3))
 (segment (start 122 108.2) (end 122 107.7) (width 0.3) (layer F.Cu) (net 3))
 (segment (start 121.95 108.25) (end 122 108.2) (width 0.3) (layer F.Cu) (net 3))
 (segment (start 124.45 108.81) (end 124.45 108.25) (width 0.3) (layer F.Cu) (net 3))
 (segment (start 124.4 108.2) (end 124.4 107.7) (width 0.3) (layer F.Cu) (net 3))
 (segment (start 124.45 108.25) (end 124.4 108.2) (width 0.3) (layer F.Cu) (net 3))
 (via (at 124 109.6) (size 0.8) (drill 0.4) (layers F.Cu B.Cu) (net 17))
 (segment (start 123.95 109.55) (end 124 109.6) (width 0.25) (layer F.Cu) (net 17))
 (segment (start 123.95 108.81) (end 123.95 109.55) (width 0.25) (layer F.Cu) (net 17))
 (segment (start 124.175 109.775) (end 124 109.6) (width 0.25) (layer B.Cu) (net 17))
 (segment (start 124.175 110.8) (end 124.175 109.775) (width 0.25) (layer B.Cu) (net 17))
 (segment (start 122.4 107) (end 122.4 106.5) (width 0.25) (layer B.Cu) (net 25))
 (segment (start 122.225 106.325) (end 122.225 105.2) (width 0.25) (layer B.Cu) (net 25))
 (segment (start 122.4 106.5) (end 122.225 106.325) (width 0.25) (layer B.Cu) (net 25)))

